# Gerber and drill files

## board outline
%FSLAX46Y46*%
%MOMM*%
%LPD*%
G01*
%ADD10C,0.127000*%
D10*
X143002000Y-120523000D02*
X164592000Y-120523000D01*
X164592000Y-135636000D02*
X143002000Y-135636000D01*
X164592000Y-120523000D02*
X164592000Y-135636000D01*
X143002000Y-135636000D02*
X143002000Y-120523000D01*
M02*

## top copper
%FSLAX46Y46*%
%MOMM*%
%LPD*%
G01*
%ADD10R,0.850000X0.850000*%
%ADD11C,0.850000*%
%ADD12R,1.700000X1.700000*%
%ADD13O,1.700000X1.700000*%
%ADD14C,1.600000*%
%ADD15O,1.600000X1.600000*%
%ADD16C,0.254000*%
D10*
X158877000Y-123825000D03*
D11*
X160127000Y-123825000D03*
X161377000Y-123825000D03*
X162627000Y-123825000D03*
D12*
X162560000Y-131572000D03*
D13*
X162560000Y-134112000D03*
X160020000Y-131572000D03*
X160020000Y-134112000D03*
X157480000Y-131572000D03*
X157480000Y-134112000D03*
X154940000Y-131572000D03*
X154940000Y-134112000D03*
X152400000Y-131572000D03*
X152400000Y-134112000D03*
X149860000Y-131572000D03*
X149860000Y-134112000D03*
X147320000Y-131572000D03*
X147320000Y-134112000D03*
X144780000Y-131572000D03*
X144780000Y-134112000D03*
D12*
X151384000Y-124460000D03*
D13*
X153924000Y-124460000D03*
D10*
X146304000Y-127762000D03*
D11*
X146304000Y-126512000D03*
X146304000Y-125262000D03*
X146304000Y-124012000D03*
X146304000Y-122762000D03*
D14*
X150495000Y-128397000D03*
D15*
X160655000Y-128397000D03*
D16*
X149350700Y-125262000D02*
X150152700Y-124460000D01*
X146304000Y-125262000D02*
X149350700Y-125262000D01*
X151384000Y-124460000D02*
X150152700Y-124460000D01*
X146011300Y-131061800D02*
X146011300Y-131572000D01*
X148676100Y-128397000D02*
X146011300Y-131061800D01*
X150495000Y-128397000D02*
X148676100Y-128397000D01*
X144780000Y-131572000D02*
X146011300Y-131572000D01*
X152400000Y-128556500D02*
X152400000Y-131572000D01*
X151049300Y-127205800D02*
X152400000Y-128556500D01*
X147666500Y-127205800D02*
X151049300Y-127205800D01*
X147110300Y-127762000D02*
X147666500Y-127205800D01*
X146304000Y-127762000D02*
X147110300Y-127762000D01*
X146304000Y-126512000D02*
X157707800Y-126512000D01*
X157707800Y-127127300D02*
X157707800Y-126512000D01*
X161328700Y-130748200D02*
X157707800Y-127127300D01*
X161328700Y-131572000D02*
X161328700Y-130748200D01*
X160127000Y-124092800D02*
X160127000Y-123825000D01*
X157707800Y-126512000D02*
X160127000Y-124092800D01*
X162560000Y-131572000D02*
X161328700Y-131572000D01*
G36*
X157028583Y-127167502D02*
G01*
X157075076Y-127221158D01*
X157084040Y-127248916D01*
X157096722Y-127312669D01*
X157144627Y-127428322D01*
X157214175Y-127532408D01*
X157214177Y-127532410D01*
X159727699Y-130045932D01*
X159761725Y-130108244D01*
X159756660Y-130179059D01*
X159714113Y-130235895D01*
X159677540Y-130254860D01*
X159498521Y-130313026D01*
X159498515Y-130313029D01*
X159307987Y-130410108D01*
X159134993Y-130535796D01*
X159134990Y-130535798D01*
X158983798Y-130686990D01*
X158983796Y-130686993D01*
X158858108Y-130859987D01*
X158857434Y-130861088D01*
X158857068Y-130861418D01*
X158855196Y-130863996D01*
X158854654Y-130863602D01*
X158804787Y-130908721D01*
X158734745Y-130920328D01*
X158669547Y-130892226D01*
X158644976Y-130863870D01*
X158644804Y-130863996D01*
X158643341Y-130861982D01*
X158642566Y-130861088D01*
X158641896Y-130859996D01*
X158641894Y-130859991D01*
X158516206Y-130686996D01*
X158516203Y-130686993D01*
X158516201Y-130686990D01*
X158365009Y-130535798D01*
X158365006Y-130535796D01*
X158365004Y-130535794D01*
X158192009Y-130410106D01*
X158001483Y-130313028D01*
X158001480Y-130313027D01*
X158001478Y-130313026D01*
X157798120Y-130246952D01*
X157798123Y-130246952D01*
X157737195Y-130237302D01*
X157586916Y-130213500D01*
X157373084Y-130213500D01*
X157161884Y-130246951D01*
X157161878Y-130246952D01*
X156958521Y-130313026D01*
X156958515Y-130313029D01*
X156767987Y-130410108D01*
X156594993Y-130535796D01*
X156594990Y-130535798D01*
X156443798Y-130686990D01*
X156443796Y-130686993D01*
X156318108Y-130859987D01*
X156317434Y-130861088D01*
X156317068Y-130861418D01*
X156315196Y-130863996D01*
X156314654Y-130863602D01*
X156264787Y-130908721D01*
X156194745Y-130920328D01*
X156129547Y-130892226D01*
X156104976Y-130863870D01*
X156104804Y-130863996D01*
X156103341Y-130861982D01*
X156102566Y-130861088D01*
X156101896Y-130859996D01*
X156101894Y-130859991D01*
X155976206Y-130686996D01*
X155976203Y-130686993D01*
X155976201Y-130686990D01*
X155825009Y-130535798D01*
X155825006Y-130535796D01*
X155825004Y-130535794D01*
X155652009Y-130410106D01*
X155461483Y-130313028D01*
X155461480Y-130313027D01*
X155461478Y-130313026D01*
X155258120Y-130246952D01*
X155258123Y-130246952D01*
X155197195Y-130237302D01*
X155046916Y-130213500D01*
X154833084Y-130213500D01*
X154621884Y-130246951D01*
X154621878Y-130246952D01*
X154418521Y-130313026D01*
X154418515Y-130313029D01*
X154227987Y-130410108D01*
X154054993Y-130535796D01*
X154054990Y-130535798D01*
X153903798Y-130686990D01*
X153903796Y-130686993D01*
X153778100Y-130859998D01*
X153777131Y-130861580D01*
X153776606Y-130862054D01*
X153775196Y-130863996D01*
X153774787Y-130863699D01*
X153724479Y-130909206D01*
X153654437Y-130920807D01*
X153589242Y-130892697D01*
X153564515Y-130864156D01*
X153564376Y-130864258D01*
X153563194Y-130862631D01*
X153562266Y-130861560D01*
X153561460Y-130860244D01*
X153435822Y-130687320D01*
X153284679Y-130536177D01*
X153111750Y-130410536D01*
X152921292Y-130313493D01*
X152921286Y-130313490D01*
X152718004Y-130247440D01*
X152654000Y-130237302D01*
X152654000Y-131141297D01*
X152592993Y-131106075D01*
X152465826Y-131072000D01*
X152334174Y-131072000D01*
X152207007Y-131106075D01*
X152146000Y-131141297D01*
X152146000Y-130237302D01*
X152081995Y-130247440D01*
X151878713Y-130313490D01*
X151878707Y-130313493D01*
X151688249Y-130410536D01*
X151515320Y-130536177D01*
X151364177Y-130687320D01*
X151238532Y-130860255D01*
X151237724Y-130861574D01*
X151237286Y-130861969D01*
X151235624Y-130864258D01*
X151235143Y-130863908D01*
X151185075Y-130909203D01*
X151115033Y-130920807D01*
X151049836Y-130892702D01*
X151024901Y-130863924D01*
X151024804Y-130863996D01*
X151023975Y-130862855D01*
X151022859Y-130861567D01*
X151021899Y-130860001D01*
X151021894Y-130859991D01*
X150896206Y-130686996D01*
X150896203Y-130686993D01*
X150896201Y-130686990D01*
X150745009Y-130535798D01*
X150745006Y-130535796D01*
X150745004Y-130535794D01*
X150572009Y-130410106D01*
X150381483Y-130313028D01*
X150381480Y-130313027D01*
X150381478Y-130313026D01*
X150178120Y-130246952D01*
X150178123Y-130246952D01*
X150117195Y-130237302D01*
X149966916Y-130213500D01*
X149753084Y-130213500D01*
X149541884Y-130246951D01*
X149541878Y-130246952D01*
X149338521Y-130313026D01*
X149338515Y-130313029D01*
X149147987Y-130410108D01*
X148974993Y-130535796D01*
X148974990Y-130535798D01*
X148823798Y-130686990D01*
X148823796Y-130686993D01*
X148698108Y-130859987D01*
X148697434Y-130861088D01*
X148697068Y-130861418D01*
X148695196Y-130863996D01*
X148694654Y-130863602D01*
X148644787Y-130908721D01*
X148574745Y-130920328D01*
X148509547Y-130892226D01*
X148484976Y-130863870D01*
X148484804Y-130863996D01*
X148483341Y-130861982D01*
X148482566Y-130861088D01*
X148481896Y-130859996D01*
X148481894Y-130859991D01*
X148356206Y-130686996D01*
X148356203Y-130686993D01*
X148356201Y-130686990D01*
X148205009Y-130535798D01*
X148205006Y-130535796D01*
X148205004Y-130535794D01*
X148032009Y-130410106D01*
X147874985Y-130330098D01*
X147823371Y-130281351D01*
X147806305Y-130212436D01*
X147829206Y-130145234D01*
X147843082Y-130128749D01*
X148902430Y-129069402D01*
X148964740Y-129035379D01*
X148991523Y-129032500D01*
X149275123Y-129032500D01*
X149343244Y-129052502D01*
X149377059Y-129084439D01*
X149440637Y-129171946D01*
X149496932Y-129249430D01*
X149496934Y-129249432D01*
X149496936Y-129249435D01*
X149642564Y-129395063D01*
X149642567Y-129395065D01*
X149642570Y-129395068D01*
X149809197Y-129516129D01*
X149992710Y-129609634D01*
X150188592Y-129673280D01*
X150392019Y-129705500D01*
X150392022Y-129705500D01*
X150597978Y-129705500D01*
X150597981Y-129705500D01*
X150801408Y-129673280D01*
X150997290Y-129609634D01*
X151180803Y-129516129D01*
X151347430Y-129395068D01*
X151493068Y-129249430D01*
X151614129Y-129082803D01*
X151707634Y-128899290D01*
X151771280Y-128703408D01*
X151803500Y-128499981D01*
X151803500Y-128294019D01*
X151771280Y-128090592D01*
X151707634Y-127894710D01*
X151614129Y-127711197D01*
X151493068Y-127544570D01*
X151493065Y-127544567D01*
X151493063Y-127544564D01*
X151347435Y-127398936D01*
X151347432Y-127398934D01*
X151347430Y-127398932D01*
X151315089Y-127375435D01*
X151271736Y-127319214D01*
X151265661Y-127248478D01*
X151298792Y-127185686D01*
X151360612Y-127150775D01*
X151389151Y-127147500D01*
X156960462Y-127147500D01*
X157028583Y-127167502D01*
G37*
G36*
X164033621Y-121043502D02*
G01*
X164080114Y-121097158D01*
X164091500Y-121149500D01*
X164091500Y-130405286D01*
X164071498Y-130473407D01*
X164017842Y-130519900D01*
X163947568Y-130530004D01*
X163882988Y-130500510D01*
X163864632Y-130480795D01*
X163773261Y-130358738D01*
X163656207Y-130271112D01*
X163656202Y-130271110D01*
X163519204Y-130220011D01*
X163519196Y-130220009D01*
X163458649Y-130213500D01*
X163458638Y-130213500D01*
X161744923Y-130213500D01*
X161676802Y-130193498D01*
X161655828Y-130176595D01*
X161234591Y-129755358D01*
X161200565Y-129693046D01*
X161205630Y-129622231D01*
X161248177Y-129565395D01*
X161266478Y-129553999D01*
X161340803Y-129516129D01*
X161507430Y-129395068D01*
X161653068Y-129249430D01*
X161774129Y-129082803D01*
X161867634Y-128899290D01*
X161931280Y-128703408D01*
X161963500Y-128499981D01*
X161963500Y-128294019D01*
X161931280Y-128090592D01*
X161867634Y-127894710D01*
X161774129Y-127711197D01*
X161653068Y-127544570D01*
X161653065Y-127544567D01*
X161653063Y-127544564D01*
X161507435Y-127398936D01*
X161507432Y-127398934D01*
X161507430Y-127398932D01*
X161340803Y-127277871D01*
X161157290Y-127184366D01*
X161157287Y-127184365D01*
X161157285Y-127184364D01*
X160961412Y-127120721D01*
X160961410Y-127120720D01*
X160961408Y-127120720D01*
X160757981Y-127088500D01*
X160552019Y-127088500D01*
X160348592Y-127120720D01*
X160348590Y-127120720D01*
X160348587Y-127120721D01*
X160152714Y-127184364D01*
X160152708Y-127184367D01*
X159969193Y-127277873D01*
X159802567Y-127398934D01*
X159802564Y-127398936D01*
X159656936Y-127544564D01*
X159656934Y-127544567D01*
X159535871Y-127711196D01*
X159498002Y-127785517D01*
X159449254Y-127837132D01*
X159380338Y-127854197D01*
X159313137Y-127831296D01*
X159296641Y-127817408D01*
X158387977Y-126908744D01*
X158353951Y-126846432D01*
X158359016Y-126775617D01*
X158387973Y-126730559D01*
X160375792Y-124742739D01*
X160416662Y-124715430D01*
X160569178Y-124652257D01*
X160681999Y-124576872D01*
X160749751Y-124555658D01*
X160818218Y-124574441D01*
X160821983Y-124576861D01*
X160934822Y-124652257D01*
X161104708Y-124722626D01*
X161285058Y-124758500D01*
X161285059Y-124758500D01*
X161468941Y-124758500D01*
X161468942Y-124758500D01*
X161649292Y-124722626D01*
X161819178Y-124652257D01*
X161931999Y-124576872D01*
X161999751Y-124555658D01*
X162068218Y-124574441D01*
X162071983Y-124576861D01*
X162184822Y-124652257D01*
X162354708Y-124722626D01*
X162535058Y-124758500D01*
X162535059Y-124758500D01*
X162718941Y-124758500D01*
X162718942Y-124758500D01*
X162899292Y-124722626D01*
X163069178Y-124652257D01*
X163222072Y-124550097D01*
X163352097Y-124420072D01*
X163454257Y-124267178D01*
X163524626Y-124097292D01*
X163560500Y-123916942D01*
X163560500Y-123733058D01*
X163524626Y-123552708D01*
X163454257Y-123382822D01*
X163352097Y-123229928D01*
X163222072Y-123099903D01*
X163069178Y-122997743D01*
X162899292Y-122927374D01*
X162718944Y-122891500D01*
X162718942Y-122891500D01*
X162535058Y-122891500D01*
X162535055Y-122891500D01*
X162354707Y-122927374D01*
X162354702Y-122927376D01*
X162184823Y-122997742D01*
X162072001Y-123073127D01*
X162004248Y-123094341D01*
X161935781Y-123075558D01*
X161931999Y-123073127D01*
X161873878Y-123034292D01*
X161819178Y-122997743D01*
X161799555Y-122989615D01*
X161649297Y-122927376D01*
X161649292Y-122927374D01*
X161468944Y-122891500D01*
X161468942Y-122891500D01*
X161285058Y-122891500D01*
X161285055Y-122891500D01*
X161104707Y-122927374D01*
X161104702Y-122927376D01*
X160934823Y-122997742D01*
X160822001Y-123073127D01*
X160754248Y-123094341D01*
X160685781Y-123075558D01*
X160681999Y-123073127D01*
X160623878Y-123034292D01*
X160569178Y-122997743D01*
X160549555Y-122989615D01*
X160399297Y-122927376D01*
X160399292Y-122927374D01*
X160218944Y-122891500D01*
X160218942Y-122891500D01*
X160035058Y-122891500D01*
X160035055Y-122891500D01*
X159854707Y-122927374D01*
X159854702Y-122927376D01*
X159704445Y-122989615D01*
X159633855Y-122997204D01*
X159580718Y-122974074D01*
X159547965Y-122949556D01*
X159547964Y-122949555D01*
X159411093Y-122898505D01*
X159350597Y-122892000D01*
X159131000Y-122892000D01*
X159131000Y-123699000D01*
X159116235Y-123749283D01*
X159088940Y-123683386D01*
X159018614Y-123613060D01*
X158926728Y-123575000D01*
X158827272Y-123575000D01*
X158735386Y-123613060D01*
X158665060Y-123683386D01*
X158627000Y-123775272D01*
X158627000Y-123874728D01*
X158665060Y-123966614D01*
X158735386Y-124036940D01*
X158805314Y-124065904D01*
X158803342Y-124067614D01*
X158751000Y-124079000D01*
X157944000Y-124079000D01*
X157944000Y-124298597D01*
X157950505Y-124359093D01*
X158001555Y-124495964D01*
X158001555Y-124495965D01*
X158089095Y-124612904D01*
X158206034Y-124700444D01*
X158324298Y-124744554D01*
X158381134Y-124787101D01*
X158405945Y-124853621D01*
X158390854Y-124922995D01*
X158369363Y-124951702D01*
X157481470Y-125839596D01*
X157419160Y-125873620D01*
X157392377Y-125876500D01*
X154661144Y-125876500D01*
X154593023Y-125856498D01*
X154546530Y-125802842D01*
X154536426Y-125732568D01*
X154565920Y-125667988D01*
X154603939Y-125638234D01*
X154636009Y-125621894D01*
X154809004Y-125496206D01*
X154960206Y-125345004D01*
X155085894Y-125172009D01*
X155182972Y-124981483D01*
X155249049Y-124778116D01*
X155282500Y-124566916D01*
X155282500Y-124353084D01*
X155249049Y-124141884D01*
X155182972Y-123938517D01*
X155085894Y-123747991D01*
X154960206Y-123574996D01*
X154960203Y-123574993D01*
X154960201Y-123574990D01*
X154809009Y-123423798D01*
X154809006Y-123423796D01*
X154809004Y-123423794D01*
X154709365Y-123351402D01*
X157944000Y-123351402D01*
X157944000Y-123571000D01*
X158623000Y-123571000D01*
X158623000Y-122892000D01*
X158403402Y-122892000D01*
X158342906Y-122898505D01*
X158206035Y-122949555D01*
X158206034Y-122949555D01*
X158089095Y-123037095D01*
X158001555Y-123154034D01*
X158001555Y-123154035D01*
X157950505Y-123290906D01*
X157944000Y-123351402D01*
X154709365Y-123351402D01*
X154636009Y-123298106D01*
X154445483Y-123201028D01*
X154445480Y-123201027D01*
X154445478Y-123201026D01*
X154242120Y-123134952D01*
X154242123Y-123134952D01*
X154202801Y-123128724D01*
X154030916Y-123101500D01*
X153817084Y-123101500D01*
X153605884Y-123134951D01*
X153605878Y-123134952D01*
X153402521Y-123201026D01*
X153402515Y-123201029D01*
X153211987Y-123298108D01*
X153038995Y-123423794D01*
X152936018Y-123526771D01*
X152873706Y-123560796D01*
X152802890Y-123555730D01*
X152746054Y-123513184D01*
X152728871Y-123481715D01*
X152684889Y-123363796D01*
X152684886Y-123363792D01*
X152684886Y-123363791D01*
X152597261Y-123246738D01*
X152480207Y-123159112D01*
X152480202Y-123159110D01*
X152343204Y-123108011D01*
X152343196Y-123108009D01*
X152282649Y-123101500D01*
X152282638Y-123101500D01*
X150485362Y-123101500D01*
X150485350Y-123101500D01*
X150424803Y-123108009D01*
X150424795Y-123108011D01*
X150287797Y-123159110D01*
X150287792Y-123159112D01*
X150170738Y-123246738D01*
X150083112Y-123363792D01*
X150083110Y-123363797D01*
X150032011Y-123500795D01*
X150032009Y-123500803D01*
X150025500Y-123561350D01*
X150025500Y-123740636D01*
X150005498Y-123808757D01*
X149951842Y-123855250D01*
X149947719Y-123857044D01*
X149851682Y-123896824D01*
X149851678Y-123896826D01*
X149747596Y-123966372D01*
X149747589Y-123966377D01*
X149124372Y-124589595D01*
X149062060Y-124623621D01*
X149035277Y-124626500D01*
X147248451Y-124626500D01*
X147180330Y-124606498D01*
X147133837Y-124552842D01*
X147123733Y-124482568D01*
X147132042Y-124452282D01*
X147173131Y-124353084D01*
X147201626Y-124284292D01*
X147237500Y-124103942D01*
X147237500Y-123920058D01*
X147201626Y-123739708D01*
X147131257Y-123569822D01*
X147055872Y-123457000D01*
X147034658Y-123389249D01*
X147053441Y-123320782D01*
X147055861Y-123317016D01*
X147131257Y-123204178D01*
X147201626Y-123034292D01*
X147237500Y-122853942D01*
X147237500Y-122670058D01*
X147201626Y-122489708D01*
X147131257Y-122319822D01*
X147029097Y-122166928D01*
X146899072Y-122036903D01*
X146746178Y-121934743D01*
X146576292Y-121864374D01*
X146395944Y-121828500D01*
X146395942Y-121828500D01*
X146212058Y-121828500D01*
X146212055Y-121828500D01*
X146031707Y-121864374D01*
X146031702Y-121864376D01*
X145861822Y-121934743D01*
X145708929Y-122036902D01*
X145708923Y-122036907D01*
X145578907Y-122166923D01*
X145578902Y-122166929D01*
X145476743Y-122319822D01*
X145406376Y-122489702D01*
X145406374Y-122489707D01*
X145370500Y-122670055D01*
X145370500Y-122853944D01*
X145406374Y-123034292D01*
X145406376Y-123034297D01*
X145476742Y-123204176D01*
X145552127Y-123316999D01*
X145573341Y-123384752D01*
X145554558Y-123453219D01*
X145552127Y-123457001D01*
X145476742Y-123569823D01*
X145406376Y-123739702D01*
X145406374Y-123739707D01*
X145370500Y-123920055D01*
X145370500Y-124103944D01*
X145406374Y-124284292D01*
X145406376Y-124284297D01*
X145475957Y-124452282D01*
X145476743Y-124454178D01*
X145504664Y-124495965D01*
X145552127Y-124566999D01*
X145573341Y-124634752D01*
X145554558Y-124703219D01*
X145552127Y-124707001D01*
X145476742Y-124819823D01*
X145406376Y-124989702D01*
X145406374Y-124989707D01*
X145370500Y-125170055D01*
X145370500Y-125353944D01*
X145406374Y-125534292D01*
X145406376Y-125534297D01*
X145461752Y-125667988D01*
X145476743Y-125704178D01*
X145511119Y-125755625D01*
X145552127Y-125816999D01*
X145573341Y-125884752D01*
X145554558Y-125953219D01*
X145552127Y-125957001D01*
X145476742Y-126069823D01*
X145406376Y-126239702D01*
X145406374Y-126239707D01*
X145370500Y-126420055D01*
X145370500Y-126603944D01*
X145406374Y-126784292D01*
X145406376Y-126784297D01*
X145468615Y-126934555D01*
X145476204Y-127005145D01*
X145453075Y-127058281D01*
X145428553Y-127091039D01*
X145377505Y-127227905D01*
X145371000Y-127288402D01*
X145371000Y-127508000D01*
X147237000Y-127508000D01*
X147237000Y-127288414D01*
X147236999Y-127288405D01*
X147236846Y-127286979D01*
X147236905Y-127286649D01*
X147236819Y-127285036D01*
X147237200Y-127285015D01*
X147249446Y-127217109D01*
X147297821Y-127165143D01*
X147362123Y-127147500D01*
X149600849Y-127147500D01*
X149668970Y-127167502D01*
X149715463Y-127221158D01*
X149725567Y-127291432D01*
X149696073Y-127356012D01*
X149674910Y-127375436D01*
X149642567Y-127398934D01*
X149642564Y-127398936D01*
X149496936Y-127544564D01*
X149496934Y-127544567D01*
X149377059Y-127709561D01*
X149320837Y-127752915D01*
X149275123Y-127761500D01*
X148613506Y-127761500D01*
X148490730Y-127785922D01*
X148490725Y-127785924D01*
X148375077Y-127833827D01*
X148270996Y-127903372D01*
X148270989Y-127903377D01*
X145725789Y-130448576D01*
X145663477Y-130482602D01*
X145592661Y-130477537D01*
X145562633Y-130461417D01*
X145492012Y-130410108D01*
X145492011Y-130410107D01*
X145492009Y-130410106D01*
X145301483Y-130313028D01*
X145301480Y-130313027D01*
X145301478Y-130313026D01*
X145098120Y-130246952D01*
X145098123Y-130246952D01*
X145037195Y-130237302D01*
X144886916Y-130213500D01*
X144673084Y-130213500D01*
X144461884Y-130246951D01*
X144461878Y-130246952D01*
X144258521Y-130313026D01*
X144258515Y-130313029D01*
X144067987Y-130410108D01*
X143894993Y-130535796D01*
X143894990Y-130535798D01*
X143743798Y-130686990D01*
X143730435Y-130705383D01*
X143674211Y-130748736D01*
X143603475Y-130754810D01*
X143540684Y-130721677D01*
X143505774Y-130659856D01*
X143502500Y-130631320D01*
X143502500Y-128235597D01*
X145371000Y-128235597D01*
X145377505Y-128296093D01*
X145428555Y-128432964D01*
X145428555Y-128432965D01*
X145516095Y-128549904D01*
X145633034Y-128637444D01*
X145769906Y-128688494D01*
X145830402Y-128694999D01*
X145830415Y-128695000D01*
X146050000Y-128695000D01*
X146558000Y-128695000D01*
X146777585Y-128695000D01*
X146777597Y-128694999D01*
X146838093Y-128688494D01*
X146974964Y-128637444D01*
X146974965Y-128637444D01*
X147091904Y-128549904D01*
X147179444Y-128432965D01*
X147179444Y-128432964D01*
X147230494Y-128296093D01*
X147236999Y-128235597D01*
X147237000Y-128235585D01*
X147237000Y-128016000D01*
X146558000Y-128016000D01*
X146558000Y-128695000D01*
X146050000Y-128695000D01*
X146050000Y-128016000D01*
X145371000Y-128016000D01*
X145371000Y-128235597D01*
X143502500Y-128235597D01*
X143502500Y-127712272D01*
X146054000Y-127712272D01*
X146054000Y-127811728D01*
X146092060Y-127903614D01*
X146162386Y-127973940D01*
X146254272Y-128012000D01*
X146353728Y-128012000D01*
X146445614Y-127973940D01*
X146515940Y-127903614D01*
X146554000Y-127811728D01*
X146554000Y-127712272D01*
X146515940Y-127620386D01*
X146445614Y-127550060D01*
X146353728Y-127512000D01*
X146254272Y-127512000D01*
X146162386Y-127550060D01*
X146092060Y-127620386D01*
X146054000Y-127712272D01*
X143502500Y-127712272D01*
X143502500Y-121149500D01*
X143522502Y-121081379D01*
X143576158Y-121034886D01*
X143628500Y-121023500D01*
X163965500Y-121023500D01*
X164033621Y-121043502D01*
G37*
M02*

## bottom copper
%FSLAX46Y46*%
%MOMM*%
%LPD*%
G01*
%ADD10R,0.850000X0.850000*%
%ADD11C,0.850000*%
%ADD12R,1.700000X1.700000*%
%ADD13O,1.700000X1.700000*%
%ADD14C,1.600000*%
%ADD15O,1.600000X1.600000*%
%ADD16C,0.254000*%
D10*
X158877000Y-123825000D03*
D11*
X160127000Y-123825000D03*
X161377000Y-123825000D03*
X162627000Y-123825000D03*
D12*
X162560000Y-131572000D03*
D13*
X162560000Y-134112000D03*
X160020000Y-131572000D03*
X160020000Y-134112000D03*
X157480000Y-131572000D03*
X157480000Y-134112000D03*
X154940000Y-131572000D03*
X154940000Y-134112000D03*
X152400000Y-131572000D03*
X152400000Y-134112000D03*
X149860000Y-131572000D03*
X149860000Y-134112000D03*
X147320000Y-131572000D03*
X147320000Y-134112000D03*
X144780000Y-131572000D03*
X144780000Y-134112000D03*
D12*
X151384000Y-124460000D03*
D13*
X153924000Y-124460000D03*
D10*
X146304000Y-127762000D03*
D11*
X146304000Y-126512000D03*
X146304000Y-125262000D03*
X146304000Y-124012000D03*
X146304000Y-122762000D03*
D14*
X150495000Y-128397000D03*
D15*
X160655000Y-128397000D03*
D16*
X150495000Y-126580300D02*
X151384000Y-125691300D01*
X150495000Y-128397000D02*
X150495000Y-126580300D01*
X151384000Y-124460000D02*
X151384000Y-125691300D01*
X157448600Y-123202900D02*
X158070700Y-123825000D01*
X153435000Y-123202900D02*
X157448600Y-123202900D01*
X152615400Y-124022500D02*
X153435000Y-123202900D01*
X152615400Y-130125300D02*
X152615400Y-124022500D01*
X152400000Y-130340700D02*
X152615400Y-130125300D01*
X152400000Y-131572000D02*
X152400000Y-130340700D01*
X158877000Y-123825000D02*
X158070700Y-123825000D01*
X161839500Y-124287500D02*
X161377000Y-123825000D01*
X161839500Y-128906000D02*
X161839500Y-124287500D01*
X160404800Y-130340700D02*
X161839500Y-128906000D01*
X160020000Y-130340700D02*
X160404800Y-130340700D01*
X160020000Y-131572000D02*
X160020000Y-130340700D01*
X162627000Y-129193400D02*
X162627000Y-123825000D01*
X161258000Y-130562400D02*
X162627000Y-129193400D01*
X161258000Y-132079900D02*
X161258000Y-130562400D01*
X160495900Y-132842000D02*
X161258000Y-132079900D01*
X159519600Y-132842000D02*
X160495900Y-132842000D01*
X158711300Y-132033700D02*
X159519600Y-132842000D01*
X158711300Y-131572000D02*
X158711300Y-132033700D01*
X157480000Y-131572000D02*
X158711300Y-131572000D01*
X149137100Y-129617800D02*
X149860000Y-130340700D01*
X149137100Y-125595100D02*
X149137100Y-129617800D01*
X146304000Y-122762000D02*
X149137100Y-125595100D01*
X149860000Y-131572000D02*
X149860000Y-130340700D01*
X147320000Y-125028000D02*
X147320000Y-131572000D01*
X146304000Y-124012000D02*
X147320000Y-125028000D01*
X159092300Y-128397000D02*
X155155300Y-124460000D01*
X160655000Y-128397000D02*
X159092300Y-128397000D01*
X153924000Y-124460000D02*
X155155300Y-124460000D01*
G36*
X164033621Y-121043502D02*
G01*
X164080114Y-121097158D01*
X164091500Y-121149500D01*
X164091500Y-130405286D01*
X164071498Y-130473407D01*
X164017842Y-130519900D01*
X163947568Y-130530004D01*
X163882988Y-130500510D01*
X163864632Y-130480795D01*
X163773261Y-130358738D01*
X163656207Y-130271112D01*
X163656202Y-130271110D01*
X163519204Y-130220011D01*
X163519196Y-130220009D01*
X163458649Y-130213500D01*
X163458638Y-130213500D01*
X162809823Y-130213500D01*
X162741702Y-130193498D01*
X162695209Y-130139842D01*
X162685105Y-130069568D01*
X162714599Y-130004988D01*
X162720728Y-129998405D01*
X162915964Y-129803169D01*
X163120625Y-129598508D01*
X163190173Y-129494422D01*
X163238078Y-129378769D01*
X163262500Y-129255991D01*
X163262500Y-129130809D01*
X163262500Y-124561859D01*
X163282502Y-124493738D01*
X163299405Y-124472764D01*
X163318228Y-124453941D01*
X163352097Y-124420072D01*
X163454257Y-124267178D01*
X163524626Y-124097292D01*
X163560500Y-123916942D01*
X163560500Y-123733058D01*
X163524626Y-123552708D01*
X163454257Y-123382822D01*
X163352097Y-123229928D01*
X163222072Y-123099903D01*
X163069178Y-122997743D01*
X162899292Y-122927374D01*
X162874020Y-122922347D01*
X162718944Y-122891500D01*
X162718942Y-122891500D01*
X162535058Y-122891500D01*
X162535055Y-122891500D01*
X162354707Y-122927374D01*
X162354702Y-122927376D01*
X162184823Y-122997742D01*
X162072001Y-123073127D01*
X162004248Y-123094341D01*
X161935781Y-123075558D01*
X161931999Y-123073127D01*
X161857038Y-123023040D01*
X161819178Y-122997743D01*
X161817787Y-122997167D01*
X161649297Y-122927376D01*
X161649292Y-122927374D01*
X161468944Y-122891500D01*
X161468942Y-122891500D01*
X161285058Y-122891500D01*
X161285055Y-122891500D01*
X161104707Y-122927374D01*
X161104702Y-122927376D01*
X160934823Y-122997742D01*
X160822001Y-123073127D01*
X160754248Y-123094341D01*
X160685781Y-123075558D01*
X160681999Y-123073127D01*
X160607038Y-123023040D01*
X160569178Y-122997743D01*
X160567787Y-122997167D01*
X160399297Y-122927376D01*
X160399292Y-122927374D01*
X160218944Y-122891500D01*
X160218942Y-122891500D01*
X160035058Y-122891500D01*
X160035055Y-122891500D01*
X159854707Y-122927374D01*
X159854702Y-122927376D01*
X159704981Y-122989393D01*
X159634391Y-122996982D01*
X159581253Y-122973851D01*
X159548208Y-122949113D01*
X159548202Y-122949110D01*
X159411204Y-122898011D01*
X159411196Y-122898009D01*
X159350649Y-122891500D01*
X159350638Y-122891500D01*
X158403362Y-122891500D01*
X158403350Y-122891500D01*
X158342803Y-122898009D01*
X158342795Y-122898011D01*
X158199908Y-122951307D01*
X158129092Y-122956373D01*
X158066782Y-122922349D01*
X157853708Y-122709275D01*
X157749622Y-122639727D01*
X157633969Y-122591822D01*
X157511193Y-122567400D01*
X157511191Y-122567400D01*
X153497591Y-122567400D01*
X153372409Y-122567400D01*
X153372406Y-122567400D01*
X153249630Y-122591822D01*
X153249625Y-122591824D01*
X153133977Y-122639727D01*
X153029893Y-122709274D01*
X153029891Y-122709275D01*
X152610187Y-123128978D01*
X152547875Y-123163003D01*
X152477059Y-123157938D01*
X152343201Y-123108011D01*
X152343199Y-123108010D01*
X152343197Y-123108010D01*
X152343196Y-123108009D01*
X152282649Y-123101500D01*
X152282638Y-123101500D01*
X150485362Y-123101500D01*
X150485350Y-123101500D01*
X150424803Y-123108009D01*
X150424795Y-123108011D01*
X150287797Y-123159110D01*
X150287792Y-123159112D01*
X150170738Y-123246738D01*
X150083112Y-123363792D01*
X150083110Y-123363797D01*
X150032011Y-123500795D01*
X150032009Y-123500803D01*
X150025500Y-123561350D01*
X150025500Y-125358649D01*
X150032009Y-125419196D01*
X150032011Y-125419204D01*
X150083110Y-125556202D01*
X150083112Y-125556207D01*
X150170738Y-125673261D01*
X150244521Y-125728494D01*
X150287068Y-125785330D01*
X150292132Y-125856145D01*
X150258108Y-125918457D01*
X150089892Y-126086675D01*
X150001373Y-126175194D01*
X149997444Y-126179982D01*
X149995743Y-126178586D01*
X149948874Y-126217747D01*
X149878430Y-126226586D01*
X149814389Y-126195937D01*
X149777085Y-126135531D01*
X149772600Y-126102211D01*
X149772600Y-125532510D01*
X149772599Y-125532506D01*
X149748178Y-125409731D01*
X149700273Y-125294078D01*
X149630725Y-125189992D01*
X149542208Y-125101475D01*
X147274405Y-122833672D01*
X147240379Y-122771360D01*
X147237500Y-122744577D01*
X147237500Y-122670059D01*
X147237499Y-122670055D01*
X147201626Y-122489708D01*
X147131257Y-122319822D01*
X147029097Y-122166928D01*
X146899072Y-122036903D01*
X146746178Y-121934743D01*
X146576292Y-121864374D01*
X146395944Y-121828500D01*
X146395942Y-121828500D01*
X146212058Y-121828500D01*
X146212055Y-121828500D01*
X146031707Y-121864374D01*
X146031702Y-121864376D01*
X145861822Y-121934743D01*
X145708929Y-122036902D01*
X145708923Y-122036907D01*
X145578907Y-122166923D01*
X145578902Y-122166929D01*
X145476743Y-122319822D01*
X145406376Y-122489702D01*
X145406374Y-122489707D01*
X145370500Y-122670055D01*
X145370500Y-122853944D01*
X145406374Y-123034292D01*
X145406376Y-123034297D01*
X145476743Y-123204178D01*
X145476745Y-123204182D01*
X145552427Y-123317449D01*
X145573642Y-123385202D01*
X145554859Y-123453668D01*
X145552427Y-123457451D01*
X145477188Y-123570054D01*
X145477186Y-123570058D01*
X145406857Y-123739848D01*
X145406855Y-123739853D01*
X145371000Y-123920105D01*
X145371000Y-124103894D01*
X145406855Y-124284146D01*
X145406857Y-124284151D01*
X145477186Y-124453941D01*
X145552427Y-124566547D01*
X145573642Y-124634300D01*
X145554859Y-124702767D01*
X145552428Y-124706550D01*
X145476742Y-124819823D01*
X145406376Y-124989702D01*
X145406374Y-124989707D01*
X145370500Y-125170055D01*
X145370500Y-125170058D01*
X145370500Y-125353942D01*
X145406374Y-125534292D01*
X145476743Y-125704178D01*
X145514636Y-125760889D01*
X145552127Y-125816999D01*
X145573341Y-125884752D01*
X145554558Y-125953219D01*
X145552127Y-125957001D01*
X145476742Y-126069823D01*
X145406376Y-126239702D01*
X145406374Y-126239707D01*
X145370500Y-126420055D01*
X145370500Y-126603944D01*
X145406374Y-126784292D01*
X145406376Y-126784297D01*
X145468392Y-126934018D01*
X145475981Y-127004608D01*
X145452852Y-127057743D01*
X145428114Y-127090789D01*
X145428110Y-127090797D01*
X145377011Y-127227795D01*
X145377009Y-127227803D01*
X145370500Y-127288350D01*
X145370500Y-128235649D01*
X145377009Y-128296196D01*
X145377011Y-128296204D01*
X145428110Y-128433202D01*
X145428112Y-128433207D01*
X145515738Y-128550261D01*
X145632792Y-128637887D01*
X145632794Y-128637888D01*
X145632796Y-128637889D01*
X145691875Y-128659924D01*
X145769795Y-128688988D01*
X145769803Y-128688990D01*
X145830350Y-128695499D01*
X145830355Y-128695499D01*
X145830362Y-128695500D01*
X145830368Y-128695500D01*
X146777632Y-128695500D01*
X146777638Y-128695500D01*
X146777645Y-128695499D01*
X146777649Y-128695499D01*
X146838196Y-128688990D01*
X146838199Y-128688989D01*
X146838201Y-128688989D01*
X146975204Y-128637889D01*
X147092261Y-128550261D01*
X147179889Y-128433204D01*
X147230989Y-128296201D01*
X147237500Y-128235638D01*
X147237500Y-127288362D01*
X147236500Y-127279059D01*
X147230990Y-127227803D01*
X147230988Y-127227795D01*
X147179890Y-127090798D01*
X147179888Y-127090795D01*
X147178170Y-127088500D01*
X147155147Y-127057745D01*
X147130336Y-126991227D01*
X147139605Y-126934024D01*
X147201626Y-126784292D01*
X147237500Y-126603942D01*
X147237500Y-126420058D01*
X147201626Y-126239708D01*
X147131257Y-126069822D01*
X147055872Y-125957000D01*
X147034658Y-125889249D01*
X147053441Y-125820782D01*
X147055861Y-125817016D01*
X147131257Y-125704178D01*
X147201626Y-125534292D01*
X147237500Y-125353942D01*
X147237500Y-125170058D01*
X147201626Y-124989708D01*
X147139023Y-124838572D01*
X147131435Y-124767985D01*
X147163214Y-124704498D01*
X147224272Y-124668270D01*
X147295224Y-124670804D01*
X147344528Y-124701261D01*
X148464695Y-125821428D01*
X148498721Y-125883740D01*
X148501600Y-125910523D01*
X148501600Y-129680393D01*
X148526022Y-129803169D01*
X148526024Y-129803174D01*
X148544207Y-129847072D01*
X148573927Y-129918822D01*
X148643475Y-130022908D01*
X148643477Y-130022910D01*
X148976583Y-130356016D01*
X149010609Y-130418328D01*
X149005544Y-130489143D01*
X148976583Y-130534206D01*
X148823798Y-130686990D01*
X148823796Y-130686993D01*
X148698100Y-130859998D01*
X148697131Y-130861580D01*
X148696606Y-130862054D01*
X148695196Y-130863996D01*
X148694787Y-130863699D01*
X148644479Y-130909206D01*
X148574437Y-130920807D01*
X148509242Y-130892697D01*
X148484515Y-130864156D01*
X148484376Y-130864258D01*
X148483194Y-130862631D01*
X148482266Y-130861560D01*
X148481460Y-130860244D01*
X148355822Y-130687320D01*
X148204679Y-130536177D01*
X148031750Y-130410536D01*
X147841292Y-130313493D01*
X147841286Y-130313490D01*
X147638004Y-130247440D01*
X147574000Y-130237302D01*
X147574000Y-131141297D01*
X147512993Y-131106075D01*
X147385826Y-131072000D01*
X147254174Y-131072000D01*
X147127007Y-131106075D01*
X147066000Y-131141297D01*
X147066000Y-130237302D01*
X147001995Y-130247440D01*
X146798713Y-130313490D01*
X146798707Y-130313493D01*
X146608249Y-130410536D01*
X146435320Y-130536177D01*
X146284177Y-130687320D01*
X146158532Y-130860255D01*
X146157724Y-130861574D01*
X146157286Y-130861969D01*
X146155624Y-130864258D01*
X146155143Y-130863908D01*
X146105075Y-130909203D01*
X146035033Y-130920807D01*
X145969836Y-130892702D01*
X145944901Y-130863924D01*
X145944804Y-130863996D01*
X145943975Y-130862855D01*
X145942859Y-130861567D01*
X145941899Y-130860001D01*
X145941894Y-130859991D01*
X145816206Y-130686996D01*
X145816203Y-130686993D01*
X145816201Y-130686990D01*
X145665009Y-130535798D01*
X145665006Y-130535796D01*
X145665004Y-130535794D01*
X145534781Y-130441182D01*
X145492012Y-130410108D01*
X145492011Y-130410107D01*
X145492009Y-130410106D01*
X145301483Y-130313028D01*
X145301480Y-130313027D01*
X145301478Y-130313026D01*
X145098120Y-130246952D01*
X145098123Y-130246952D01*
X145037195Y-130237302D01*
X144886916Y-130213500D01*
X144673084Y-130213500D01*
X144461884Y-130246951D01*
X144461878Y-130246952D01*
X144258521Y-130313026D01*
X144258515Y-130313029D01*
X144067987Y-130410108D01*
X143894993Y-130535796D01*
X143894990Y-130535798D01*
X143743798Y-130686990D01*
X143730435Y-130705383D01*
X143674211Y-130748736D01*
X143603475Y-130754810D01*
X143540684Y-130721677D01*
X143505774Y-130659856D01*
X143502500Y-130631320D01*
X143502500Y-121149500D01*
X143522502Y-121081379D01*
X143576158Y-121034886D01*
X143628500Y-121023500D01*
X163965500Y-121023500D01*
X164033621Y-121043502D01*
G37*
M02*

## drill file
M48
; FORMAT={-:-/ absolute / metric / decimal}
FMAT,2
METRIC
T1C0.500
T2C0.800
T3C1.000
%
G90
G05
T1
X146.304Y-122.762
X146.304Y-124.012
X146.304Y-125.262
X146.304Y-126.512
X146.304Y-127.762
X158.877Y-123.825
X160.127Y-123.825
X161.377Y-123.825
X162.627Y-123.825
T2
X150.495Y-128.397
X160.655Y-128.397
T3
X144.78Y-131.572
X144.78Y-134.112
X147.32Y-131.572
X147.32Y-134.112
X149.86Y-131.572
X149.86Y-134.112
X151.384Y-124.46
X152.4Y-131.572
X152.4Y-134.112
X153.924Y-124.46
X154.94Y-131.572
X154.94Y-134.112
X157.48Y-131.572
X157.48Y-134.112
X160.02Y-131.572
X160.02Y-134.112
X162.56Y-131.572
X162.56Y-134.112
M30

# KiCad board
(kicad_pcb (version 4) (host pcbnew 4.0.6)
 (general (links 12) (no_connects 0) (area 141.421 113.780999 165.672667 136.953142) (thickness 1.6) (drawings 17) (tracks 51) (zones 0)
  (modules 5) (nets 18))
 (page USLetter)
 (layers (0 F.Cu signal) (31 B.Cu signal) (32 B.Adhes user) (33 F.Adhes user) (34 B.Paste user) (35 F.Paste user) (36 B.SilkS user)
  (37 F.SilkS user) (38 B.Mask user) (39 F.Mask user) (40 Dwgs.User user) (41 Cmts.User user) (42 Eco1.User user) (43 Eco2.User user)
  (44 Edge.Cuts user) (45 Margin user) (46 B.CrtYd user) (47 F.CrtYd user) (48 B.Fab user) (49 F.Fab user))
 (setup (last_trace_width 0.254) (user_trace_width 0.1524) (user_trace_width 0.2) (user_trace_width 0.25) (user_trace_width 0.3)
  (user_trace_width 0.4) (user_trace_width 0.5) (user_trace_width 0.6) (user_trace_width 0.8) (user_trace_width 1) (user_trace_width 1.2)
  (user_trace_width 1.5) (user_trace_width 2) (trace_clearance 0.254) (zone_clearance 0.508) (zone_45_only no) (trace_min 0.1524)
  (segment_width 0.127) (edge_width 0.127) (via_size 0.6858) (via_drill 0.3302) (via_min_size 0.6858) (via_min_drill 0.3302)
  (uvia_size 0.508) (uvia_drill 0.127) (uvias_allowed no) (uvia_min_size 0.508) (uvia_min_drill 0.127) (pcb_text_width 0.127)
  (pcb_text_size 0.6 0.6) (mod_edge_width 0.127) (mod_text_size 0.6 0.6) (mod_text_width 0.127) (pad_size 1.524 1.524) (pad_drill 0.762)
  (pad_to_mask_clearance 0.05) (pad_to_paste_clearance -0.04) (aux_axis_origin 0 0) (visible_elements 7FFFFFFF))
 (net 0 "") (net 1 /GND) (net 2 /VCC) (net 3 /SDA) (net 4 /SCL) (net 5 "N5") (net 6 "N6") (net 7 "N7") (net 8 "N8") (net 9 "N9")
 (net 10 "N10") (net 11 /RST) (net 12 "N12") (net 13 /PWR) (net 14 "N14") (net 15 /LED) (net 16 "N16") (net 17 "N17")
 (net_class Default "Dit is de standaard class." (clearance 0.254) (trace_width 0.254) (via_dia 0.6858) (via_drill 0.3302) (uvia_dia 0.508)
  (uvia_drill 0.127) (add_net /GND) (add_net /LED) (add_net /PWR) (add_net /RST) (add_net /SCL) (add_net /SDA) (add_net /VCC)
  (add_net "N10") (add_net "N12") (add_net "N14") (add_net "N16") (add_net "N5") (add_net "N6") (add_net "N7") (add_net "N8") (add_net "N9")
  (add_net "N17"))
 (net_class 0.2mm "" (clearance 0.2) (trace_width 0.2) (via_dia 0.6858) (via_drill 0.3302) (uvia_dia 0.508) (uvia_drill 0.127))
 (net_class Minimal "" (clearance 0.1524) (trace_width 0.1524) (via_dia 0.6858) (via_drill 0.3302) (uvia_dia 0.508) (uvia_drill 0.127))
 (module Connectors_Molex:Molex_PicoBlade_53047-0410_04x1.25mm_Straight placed (layer F.Cu) (at 158.877 123.825)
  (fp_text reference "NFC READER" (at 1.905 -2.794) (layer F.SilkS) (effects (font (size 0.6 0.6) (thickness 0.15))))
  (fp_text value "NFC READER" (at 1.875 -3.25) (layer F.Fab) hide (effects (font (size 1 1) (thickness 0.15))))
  (pad 1 thru_hole rect (at 0 0) (size 0.85 0.85) (drill 0.5) (layers *.Cu *.Mask) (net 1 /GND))
  (pad 2 thru_hole circle (at 1.25 0) (size 0.85 0.85) (drill 0.5) (layers *.Cu *.Mask) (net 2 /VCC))
  (pad 3 thru_hole circle (at 2.5 0) (size 0.85 0.85) (drill 0.5) (layers *.Cu *.Mask) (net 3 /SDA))
  (pad 4 thru_hole circle (at 3.75 0) (size 0.85 0.85) (drill 0.5) (layers *.Cu *.Mask) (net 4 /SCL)))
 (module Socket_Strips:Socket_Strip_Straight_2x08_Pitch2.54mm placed (layer B.Cu) (at 162.56 131.572 90)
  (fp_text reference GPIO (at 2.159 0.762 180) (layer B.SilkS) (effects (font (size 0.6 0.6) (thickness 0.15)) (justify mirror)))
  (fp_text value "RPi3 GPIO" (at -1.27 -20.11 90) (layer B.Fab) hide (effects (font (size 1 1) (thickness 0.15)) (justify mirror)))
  (pad 1 thru_hole rect (at 0 0 90) (size 1.7 1.7) (drill 1) (layers *.Cu *.Mask) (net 2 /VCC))
  (pad 2 thru_hole oval (at -2.54 0 90) (size 1.7 1.7) (drill 1) (layers *.Cu *.Mask) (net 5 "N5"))
  (pad 3 thru_hole oval (at 0 -2.54 90) (size 1.7 1.7) (drill 1) (layers *.Cu *.Mask) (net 3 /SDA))
  (pad 4 thru_hole oval (at -2.54 -2.54 90) (size 1.7 1.7) (drill 1) (layers *.Cu *.Mask) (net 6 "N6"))
  (pad 5 thru_hole oval (at 0 -5.08 90) (size 1.7 1.7) (drill 1) (layers *.Cu *.Mask) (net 4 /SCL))
  (pad 6 thru_hole oval (at -2.54 -5.08 90) (size 1.7 1.7) (drill 1) (layers *.Cu *.Mask) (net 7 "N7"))
  (pad 7 thru_hole oval (at 0 -7.62 90) (size 1.7 1.7) (drill 1) (layers *.Cu *.Mask) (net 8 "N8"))
  (pad 8 thru_hole oval (at -2.54 -7.62 90) (size 1.7 1.7) (drill 1) (layers *.Cu *.Mask) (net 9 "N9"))
  (pad 9 thru_hole oval (at 0 -10.16 90) (size 1.7 1.7) (drill 1) (layers *.Cu *.Mask) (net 1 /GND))
  (pad 10 thru_hole oval (at -2.54 -10.16 90) (size 1.7 1.7) (drill 1) (layers *.Cu *.Mask) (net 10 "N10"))
  (pad 11 thru_hole oval (at 0 -12.7 90) (size 1.7 1.7) (drill 1) (layers *.Cu *.Mask) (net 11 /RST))
  (pad 12 thru_hole oval (at -2.54 -12.7 90) (size 1.7 1.7) (drill 1) (layers *.Cu *.Mask) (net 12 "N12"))
  (pad 13 thru_hole oval (at 0 -15.24 90) (size 1.7 1.7) (drill 1) (layers *.Cu *.Mask) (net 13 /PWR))
  (pad 14 thru_hole oval (at -2.54 -15.24 90) (size 1.7 1.7) (drill 1) (layers *.Cu *.Mask) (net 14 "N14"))
  (pad 15 thru_hole oval (at 0 -17.78 90) (size 1.7 1.7) (drill 1) (layers *.Cu *.Mask) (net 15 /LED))
  (pad 16 thru_hole oval (at -2.54 -17.78 90) (size 1.7 1.7) (drill 1) (layers *.Cu *.Mask) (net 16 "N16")))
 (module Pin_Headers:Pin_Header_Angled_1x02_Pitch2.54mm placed (layer F.Cu) (at 151.384 124.46 90)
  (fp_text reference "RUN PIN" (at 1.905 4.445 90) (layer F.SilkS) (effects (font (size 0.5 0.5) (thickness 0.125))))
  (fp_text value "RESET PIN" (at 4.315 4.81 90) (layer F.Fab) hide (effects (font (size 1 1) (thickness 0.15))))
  (pad 1 thru_hole rect (at 0 0 90) (size 1.7 1.7) (drill 1) (layers *.Cu *.Mask) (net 15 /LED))
  (pad 2 thru_hole oval (at 0 2.54 90) (size 1.7 1.7) (drill 1) (layers *.Cu *.Mask) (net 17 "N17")))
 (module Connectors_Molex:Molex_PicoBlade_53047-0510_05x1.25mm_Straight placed (layer F.Cu) (at 146.304 127.762 90)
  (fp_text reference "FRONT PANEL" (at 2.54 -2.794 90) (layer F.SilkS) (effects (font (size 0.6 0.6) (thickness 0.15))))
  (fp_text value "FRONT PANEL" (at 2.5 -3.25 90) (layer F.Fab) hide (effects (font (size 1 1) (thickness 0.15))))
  (pad 1 thru_hole rect (at 0 0 90) (size 0.85 0.85) (drill 0.5) (layers *.Cu *.Mask) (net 1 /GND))
  (pad 2 thru_hole circle (at 1.25 0 90) (size 0.85 0.85) (drill 0.5) (layers *.Cu *.Mask) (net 2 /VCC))
  (pad 3 thru_hole circle (at 2.5 0 90) (size 0.85 0.85) (drill 0.5) (layers *.Cu *.Mask) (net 15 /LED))
  (pad 4 thru_hole circle (at 3.75 0 90) (size 0.85 0.85) (drill 0.5) (layers *.Cu *.Mask) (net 13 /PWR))
  (pad 5 thru_hole circle (at 5 0 90) (size 0.85 0.85) (drill 0.5) (layers *.Cu *.Mask) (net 11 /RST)))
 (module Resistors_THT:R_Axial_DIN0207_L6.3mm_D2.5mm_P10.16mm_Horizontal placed (layer F.Cu) (at 150.495 128.397)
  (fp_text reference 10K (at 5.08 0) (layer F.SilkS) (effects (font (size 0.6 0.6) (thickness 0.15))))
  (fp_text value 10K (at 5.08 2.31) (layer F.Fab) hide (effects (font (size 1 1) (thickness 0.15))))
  (pad 1 thru_hole circle (at 0 0) (size 1.6 1.6) (drill 0.8) (layers *.Cu *.Mask) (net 15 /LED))
  (pad 2 thru_hole oval (at 10.16 0) (size 1.6 1.6) (drill 0.8) (layers *.Cu *.Mask) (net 17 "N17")))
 (gr_line (start 143.002 120.523) (end 164.592 120.523) (angle 90) (layer Edge.Cuts) (width 0.127))
 (gr_line (start 164.592 135.636) (end 143.002 135.636) (angle 90) (layer Edge.Cuts) (width 0.127))
 (gr_line (start 164.592 120.523) (end 164.592 135.636) (angle 90) (layer Edge.Cuts) (width 0.127))
 (gr_line (start 143.002 135.636) (end 143.002 120.523) (angle 90) (layer Edge.Cuts) (width 0.127))
 (segment (start 149.3507 125.262) (end 150.1527 124.46) (width 0.254) (layer F.Cu) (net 15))
 (segment (start 146.304 125.262) (end 149.3507 125.262) (width 0.254) (layer F.Cu) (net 15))
 (segment (start 151.384 124.46) (end 150.1527 124.46) (width 0.254) (layer F.Cu) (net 15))
 (segment (start 146.0113 131.0618) (end 146.0113 131.572) (width 0.254) (layer F.Cu) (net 15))
 (segment (start 148.6761 128.397) (end 146.0113 131.0618) (width 0.254) (layer F.Cu) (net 15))
 (segment (start 150.495 128.397) (end 148.6761 128.397) (width 0.254) (layer F.Cu) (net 15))
 (segment (start 144.78 131.572) (end 146.0113 131.572) (width 0.254) (layer F.Cu) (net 15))
 (segment (start 150.495 126.5803) (end 151.384 125.6913) (width 0.254) (layer B.Cu) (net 15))
 (segment (start 150.495 128.397) (end 150.495 126.5803) (width 0.254) (layer B.Cu) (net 15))
 (segment (start 151.384 124.46) (end 151.384 125.6913) (width 0.254) (layer B.Cu) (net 15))
 (segment (start 152.4 128.5565) (end 152.4 131.572) (width 0.254) (layer F.Cu) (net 1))
 (segment (start 151.0493 127.2058) (end 152.4 128.5565) (width 0.254) (layer F.Cu) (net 1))
 (segment (start 147.6665 127.2058) (end 151.0493 127.2058) (width 0.254) (layer F.Cu) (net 1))
 (segment (start 147.1103 127.762) (end 147.6665 127.2058) (width 0.254) (layer F.Cu) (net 1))
 (segment (start 146.304 127.762) (end 147.1103 127.762) (width 0.254) (layer F.Cu) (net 1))
 (segment (start 157.4486 123.2029) (end 158.0707 123.825) (width 0.254) (layer B.Cu) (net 1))
 (segment (start 153.435 123.2029) (end 157.4486 123.2029) (width 0.254) (layer B.Cu) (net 1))
 (segment (start 152.6154 124.0225) (end 153.435 123.2029) (width 0.254) (layer B.Cu) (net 1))
 (segment (start 152.6154 130.1253) (end 152.6154 124.0225) (width 0.254) (layer B.Cu) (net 1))
 (segment (start 152.4 130.3407) (end 152.6154 130.1253) (width 0.254) (layer B.Cu) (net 1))
 (segment (start 152.4 131.572) (end 152.4 130.3407) (width 0.254) (layer B.Cu) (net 1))
 (segment (start 158.877 123.825) (end 158.0707 123.825) (width 0.254) (layer B.Cu) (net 1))
 (segment (start 146.304 126.512) (end 157.7078 126.512) (width 0.254) (layer F.Cu) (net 2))
 (segment (start 157.7078 127.1273) (end 157.7078 126.512) (width 0.254) (layer F.Cu) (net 2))
 (segment (start 161.3287 130.7482) (end 157.7078 127.1273) (width 0.254) (layer F.Cu) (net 2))
 (segment (start 161.3287 131.572) (end 161.3287 130.7482) (width 0.254) (layer F.Cu) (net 2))
 (segment (start 160.127 124.0928) (end 160.127 123.825) (width 0.254) (layer F.Cu) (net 2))
 (segment (start 157.7078 126.512) (end 160.127 124.0928) (width 0.254) (layer F.Cu) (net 2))
 (segment (start 162.56 131.572) (end 161.3287 131.572) (width 0.254) (layer F.Cu) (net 2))
 (segment (start 161.8395 124.2875) (end 161.377 123.825) (width 0.254) (layer B.Cu) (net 3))
 (segment (start 161.8395 128.906) (end 161.8395 124.2875) (width 0.254) (layer B.Cu) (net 3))
 (segment (start 160.4048 130.3407) (end 161.8395 128.906) (width 0.254) (layer B.Cu) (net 3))
 (segment (start 160.02 130.3407) (end 160.4048 130.3407) (width 0.254) (layer B.Cu) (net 3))
 (segment (start 160.02 131.572) (end 160.02 130.3407) (width 0.254) (layer B.Cu) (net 3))
 (segment (start 162.627 129.1934) (end 162.627 123.825) (width 0.254) (layer B.Cu) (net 4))
 (segment (start 161.258 130.5624) (end 162.627 129.1934) (width 0.254) (layer B.Cu) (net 4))
 (segment (start 161.258 132.0799) (end 161.258 130.5624) (width 0.254) (layer B.Cu) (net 4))
 (segment (start 160.4959 132.842) (end 161.258 132.0799) (width 0.254) (layer B.Cu) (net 4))
 (segment (start 159.5196 132.842) (end 160.4959 132.842) (width 0.254) (layer B.Cu) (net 4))
 (segment (start 158.7113 132.0337) (end 159.5196 132.842) (width 0.254) (layer B.Cu) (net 4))
 (segment (start 158.7113 131.572) (end 158.7113 132.0337) (width 0.254) (layer B.Cu) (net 4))
 (segment (start 157.48 131.572) (end 158.7113 131.572) (width 0.254) (layer B.Cu) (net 4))
 (segment (start 149.1371 129.6178) (end 149.86 130.3407) (width 0.254) (layer B.Cu) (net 11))
 (segment (start 149.1371 125.5951) (end 149.1371 129.6178) (width 0.254) (layer B.Cu) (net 11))
 (segment (start 146.304 122.762) (end 149.1371 125.5951) (width 0.254) (layer B.Cu) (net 11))
 (segment (start 149.86 131.572) (end 149.86 130.3407) (width 0.254) (layer B.Cu) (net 11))
 (segment (start 147.32 125.028) (end 147.32 131.572) (width 0.254) (layer B.Cu) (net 13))
 (segment (start 146.304 124.012) (end 147.32 125.028) (width 0.254) (layer B.Cu) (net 13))
 (segment (start 159.0923 128.397) (end 155.1553 124.46) (width 0.254) (layer B.Cu) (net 17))
 (segment (start 160.655 128.397) (end 159.0923 128.397) (width 0.254) (layer B.Cu) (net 17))
 (segment (start 153.924 124.46) (end 155.1553 124.46) (width 0.254) (layer B.Cu) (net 17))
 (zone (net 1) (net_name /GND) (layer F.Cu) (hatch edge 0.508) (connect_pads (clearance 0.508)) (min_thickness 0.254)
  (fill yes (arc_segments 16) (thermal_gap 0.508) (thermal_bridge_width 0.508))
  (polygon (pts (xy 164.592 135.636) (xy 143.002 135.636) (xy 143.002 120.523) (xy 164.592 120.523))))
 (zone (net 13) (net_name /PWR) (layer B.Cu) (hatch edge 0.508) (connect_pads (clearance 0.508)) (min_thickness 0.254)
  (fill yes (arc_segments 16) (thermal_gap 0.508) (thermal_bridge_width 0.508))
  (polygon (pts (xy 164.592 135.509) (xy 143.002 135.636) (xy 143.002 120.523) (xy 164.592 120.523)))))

